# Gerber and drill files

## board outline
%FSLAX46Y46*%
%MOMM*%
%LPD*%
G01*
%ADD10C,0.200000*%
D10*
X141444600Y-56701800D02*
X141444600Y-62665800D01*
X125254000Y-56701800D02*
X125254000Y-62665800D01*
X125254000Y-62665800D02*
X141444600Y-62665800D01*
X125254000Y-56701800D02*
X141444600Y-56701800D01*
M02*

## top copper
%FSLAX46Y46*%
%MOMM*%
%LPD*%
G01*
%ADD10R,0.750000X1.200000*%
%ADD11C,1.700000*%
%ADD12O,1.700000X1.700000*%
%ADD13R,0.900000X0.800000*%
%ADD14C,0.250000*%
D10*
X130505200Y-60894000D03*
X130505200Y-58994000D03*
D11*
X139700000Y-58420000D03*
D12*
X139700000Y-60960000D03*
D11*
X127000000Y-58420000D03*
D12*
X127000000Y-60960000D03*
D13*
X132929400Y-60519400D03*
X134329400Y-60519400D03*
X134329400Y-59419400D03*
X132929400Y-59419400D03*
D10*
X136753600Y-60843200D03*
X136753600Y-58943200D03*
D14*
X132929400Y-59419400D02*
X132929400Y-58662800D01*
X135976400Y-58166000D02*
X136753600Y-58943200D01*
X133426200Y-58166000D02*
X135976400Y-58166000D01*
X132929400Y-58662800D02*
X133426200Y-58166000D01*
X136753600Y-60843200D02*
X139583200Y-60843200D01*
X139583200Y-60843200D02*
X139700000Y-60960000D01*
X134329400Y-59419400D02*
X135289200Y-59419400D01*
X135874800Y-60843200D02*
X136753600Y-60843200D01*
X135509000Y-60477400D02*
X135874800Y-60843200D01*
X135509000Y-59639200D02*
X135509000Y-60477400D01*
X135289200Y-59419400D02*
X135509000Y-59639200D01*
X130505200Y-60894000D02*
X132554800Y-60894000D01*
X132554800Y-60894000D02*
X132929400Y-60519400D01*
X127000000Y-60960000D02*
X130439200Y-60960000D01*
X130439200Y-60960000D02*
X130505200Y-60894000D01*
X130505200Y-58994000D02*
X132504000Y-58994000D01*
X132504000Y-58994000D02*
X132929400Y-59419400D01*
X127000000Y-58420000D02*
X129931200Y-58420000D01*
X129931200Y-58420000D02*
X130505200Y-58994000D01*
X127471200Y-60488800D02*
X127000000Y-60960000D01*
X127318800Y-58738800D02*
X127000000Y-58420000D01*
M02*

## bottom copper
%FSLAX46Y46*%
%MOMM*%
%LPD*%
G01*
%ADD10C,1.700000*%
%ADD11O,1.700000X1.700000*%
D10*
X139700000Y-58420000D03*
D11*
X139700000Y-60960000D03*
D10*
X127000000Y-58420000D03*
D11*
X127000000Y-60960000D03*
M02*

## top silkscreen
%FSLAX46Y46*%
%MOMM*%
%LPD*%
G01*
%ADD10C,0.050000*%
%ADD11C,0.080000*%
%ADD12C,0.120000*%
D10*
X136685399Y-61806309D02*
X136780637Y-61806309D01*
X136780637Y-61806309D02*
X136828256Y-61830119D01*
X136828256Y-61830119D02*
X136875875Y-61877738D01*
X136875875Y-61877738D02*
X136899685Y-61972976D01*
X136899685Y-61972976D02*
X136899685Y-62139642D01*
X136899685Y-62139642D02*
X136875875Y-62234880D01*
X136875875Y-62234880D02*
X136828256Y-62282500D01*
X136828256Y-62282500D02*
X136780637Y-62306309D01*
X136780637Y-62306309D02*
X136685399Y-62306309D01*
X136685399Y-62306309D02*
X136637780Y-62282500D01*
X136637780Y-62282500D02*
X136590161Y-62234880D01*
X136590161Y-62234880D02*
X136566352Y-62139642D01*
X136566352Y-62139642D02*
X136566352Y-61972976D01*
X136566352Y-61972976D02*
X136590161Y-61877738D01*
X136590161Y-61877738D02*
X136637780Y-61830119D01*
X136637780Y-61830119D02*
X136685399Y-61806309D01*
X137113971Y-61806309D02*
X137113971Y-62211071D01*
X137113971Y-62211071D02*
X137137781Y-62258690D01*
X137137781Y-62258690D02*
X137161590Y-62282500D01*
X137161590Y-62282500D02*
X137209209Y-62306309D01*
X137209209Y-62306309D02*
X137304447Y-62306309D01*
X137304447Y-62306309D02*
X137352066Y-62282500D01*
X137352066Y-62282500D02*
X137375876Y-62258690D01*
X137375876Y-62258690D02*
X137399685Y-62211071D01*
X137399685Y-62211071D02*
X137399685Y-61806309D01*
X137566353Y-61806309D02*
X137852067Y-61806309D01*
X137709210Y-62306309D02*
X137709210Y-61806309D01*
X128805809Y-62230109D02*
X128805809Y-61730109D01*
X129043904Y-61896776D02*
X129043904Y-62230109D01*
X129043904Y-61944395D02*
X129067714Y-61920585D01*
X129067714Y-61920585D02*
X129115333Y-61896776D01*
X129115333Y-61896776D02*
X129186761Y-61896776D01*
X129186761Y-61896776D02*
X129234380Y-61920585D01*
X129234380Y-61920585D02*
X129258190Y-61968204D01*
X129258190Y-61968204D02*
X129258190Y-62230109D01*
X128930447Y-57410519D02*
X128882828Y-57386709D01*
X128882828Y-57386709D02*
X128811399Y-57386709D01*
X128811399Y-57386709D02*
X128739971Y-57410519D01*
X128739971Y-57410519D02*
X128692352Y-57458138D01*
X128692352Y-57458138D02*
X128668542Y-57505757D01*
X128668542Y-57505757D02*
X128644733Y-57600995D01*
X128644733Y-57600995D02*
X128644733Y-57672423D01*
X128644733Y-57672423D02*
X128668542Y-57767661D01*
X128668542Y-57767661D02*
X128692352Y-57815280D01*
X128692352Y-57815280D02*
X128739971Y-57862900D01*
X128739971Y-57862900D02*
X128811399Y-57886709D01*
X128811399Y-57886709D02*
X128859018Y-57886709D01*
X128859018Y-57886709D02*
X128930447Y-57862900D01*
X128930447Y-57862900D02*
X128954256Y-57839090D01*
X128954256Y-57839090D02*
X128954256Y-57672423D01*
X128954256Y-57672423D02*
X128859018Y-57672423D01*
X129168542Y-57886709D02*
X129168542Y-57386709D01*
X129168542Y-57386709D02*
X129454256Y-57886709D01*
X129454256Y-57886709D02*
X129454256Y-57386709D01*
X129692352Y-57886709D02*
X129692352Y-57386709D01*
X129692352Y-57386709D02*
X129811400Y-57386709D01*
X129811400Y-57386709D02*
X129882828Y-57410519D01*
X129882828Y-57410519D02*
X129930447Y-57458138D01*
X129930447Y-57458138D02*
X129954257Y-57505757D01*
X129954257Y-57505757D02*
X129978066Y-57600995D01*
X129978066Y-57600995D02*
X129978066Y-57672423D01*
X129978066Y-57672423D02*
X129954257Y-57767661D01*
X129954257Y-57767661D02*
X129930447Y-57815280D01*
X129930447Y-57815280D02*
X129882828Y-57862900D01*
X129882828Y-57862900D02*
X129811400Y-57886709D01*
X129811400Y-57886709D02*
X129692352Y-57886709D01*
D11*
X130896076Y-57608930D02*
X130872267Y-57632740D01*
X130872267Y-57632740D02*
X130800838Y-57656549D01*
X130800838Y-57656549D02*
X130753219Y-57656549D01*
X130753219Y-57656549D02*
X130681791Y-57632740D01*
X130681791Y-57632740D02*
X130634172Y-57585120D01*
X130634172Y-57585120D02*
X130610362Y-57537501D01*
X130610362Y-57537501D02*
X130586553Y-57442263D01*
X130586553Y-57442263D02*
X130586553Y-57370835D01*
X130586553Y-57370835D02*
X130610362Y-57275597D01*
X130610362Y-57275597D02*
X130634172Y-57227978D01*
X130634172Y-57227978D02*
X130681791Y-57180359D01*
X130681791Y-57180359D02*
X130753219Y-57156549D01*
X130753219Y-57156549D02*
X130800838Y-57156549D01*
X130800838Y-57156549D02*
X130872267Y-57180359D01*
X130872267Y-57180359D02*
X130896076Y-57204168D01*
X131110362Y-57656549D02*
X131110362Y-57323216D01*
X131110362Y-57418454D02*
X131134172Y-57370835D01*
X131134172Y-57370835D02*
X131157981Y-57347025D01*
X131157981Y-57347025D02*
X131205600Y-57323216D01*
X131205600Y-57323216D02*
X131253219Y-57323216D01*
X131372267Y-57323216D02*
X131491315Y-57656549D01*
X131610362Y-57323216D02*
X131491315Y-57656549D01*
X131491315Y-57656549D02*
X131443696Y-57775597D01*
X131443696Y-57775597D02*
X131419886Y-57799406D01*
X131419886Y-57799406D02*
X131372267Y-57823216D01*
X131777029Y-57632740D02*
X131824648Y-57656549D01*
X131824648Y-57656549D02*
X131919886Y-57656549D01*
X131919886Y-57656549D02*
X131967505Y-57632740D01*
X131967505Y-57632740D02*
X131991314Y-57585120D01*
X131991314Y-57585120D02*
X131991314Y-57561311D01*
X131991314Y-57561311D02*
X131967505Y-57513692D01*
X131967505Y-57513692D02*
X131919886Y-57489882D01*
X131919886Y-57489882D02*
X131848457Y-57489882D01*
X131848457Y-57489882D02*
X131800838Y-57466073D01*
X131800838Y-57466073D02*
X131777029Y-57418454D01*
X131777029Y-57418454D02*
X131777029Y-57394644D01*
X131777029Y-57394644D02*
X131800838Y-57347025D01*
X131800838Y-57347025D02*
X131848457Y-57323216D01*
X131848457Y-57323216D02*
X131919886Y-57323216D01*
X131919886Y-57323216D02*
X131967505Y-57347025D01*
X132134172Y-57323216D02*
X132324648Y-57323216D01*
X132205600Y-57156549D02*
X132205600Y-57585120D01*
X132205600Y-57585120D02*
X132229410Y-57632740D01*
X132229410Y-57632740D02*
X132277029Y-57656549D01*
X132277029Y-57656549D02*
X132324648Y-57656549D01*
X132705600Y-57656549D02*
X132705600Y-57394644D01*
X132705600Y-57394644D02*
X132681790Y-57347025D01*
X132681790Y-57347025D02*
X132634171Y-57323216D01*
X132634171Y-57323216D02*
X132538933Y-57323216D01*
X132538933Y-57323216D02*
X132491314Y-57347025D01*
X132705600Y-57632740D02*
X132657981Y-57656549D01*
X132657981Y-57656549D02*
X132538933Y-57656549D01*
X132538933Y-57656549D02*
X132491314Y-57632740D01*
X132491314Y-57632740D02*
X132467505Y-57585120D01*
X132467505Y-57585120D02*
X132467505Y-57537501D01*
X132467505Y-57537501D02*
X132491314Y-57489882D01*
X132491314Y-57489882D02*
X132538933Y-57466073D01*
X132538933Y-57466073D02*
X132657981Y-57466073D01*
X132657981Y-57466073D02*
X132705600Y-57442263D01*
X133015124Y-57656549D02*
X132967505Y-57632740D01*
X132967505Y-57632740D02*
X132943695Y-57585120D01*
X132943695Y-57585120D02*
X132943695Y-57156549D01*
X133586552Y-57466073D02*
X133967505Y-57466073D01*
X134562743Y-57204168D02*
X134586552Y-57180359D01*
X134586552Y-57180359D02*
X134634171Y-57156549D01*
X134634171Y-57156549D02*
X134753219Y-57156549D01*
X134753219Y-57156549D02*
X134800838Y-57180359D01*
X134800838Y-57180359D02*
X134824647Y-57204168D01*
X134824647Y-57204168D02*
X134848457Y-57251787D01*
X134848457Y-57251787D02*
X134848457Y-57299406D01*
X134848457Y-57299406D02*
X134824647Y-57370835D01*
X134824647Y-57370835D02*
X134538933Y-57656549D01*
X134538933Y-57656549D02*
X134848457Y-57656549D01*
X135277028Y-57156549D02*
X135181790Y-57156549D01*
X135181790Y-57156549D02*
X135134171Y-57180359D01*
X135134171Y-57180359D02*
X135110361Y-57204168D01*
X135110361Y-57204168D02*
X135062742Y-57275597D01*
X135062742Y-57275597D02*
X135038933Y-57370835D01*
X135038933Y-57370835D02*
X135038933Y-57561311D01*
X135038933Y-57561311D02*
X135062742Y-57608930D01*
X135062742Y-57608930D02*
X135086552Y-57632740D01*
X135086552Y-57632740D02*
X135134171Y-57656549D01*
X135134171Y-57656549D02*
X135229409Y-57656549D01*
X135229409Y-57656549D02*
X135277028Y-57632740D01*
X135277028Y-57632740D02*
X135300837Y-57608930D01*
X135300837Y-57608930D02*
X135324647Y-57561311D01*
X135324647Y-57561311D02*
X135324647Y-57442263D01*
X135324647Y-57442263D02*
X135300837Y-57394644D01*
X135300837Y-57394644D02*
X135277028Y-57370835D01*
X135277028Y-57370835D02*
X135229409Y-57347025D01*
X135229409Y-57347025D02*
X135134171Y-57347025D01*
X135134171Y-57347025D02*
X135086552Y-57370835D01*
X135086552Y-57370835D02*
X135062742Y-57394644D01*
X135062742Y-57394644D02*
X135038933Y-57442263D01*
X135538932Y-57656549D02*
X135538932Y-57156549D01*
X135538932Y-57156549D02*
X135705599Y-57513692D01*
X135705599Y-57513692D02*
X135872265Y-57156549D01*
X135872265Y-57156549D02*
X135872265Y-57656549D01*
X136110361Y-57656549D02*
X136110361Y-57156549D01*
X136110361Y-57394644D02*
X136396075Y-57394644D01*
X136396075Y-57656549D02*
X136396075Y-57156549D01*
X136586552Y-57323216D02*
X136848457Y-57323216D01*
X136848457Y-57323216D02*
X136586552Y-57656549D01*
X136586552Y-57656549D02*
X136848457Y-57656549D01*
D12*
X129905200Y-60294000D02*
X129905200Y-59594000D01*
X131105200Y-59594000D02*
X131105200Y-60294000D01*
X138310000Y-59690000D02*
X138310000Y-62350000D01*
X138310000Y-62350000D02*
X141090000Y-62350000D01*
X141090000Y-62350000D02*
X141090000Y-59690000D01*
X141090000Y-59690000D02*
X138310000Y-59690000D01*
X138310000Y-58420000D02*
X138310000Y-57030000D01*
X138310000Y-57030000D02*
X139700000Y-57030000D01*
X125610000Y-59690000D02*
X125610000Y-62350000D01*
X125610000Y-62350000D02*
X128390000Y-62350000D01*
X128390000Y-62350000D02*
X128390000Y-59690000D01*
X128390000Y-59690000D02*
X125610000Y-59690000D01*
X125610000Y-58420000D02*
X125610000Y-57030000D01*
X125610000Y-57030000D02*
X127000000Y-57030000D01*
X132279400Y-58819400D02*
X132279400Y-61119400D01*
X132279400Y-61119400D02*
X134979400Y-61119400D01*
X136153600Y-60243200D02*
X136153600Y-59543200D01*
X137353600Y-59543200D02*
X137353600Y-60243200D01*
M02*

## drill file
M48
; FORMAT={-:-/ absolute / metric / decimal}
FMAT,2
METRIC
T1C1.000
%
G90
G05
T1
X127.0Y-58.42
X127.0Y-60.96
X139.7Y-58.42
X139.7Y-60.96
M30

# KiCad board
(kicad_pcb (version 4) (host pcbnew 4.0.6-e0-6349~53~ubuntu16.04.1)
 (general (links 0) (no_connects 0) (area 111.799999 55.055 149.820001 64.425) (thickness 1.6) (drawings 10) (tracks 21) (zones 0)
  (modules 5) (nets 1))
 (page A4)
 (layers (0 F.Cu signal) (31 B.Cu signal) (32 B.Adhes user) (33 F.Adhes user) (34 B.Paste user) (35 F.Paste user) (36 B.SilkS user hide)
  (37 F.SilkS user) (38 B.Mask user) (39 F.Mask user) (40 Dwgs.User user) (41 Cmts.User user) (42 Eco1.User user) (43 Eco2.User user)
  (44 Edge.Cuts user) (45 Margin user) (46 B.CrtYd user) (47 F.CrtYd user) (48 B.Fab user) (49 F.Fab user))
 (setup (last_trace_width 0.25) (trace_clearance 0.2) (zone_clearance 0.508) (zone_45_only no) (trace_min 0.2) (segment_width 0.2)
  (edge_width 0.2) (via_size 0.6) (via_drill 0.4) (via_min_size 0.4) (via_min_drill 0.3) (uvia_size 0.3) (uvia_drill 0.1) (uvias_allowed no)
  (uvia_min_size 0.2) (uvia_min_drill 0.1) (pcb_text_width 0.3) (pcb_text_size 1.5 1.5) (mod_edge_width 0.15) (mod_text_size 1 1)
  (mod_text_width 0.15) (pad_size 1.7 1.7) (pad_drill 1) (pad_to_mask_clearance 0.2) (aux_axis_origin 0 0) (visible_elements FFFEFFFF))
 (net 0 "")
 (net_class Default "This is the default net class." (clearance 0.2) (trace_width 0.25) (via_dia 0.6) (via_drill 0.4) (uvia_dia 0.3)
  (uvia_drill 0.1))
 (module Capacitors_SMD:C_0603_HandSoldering (layer F.Cu) (at 130.5052 59.944 90)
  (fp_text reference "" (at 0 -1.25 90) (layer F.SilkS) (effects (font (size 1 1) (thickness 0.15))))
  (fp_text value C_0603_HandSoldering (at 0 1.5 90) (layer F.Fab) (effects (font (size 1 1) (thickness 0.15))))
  (fp_line (start -0.35 -0.6) (end 0.35 -0.6) (layer F.SilkS) (width 0.12))
  (fp_line (start 0.35 0.6) (end -0.35 0.6) (layer F.SilkS) (width 0.12))
  (pad 1 smd rect (at -0.95 0 90) (size 1.2 0.75) (layers F.Cu F.Paste F.Mask))
  (pad 2 smd rect (at 0.95 0 90) (size 1.2 0.75) (layers F.Cu F.Paste F.Mask)))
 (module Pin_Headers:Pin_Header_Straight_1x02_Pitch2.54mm (layer F.Cu) (at 139.7 58.42)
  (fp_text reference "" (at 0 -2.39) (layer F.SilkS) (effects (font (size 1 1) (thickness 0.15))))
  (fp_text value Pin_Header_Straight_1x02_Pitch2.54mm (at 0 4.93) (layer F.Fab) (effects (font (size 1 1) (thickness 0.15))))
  (fp_line (start -1.39 1.27) (end -1.39 3.93) (layer F.SilkS) (width 0.12))
  (fp_line (start -1.39 3.93) (end 1.39 3.93) (layer F.SilkS) (width 0.12))
  (fp_line (start 1.39 3.93) (end 1.39 1.27) (layer F.SilkS) (width 0.12))
  (fp_line (start 1.39 1.27) (end -1.39 1.27) (layer F.SilkS) (width 0.12))
  (fp_line (start -1.39 0) (end -1.39 -1.39) (layer F.SilkS) (width 0.12))
  (fp_line (start -1.39 -1.39) (end 0 -1.39) (layer F.SilkS) (width 0.12))
  (pad 1 thru_hole circle (at 0 0) (size 1.7 1.7) (drill 1) (layers *.Cu *.Mask))
  (pad 2 thru_hole oval (at 0 2.54) (size 1.7 1.7) (drill 1) (layers *.Cu *.Mask)))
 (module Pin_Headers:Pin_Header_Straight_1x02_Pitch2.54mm (layer F.Cu) (at 127 58.42)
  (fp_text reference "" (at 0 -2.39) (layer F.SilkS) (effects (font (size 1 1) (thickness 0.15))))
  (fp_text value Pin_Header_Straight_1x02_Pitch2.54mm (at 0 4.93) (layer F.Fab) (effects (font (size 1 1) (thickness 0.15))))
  (fp_line (start -1.39 1.27) (end -1.39 3.93) (layer F.SilkS) (width 0.12))
  (fp_line (start -1.39 3.93) (end 1.39 3.93) (layer F.SilkS) (width 0.12))
  (fp_line (start 1.39 3.93) (end 1.39 1.27) (layer F.SilkS) (width 0.12))
  (fp_line (start 1.39 1.27) (end -1.39 1.27) (layer F.SilkS) (width 0.12))
  (fp_line (start -1.39 0) (end -1.39 -1.39) (layer F.SilkS) (width 0.12))
  (fp_line (start -1.39 -1.39) (end 0 -1.39) (layer F.SilkS) (width 0.12))
  (pad 1 thru_hole circle (at 0 0) (size 1.7 1.7) (drill 1) (layers *.Cu *.Mask))
  (pad 2 thru_hole oval (at 0 2.54) (size 1.7 1.7) (drill 1) (layers *.Cu *.Mask)))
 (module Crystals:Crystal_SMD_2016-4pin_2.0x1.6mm (layer F.Cu) (at 133.6294 59.9694)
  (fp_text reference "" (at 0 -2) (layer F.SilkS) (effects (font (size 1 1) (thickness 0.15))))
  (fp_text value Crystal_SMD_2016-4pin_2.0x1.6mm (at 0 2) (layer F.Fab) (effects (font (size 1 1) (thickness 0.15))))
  (fp_line (start -1.35 -1.15) (end -1.35 1.15) (layer F.SilkS) (width 0.12))
  (fp_line (start -1.35 1.15) (end 1.35 1.15) (layer F.SilkS) (width 0.12))
  (pad 1 smd rect (at -0.7 0.55) (size 0.9 0.8) (layers F.Cu F.Paste F.Mask))
  (pad 2 smd rect (at 0.7 0.55) (size 0.9 0.8) (layers F.Cu F.Paste F.Mask))
  (pad 3 smd rect (at 0.7 -0.55) (size 0.9 0.8) (layers F.Cu F.Paste F.Mask))
  (pad 4 smd rect (at -0.7 -0.55) (size 0.9 0.8) (layers F.Cu F.Paste F.Mask)))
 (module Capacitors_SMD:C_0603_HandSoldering (layer F.Cu) (at 136.7536 59.8932 90)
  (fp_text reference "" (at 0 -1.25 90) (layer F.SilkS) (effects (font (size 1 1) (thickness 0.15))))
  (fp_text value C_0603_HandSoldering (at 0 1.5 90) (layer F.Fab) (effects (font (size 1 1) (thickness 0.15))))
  (fp_line (start -0.35 -0.6) (end 0.35 -0.6) (layer F.SilkS) (width 0.12))
  (fp_line (start 0.35 0.6) (end -0.35 0.6) (layer F.SilkS) (width 0.12))
  (pad 1 smd rect (at -0.95 0 90) (size 1.2 0.75) (layers F.Cu F.Paste F.Mask))
  (pad 2 smd rect (at 0.95 0 90) (size 1.2 0.75) (layers F.Cu F.Paste F.Mask)))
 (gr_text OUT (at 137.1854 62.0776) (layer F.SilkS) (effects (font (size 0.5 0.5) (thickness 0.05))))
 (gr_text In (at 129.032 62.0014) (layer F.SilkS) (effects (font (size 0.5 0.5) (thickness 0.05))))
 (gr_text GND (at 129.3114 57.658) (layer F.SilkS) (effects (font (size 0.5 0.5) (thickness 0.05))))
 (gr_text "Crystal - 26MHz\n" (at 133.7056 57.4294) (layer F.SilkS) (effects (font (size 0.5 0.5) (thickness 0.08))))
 (gr_line (start 141.4446 56.7018) (end 141.4446 62.6658) (angle 90) (layer Edge.Cuts) (width 0.2))
 (gr_line (start 125.254 56.7018) (end 125.254 62.6658) (angle 90) (layer Edge.Cuts) (width 0.2))
 (gr_line (start 125.254 62.6658) (end 141.4446 62.6658) (angle 90) (layer Edge.Cuts) (width 0.2))
 (gr_line (start 125.254 56.7018) (end 141.4446 56.7018) (angle 90) (layer Edge.Cuts) (width 0.2))
 (segment (start 132.9294 59.4194) (end 132.9294 58.6628) (width 0.25) (layer F.Cu) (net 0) (status 400000))
 (segment (start 135.9764 58.166) (end 136.7536 58.9432) (width 0.25) (layer F.Cu) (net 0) (status 800000))
 (segment (start 133.4262 58.166) (end 135.9764 58.166) (width 0.25) (layer F.Cu) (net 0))
 (segment (start 132.9294 58.6628) (end 133.4262 58.166) (width 0.25) (layer F.Cu) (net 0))
 (segment (start 136.7536 60.8432) (end 139.5832 60.8432) (width 0.25) (layer F.Cu) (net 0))
 (segment (start 139.5832 60.8432) (end 139.7 60.96) (width 0.25) (layer F.Cu) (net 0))
 (segment (start 134.3294 59.4194) (end 135.2892 59.4194) (width 0.25) (layer F.Cu) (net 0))
 (segment (start 135.8748 60.8432) (end 136.7536 60.8432) (width 0.25) (layer F.Cu) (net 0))
 (segment (start 135.509 60.4774) (end 135.8748 60.8432) (width 0.25) (layer F.Cu) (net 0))
 (segment (start 135.509 59.6392) (end 135.509 60.4774) (width 0.25) (layer F.Cu) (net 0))
 (segment (start 135.2892 59.4194) (end 135.509 59.6392) (width 0.25) (layer F.Cu) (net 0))
 (segment (start 130.5052 60.894) (end 132.5548 60.894) (width 0.25) (layer F.Cu) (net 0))
 (segment (start 132.5548 60.894) (end 132.9294 60.5194) (width 0.25) (layer F.Cu) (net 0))
 (segment (start 127 60.96) (end 130.4392 60.96) (width 0.25) (layer F.Cu) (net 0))
 (segment (start 130.4392 60.96) (end 130.5052 60.894) (width 0.25) (layer F.Cu) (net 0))
 (segment (start 130.5052 58.994) (end 132.504 58.994) (width 0.25) (layer F.Cu) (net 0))
 (segment (start 132.504 58.994) (end 132.9294 59.4194) (width 0.25) (layer F.Cu) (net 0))
 (segment (start 127 58.42) (end 129.9312 58.42) (width 0.25) (layer F.Cu) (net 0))
 (segment (start 129.9312 58.42) (end 130.5052 58.994) (width 0.25) (layer F.Cu) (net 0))
 (segment (start 127.4712 60.4888) (end 127 60.96) (width 0.25) (layer F.Cu) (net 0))
 (segment (start 127.3188 58.7388) (end 127 58.42) (width 0.25) (layer F.Cu) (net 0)))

